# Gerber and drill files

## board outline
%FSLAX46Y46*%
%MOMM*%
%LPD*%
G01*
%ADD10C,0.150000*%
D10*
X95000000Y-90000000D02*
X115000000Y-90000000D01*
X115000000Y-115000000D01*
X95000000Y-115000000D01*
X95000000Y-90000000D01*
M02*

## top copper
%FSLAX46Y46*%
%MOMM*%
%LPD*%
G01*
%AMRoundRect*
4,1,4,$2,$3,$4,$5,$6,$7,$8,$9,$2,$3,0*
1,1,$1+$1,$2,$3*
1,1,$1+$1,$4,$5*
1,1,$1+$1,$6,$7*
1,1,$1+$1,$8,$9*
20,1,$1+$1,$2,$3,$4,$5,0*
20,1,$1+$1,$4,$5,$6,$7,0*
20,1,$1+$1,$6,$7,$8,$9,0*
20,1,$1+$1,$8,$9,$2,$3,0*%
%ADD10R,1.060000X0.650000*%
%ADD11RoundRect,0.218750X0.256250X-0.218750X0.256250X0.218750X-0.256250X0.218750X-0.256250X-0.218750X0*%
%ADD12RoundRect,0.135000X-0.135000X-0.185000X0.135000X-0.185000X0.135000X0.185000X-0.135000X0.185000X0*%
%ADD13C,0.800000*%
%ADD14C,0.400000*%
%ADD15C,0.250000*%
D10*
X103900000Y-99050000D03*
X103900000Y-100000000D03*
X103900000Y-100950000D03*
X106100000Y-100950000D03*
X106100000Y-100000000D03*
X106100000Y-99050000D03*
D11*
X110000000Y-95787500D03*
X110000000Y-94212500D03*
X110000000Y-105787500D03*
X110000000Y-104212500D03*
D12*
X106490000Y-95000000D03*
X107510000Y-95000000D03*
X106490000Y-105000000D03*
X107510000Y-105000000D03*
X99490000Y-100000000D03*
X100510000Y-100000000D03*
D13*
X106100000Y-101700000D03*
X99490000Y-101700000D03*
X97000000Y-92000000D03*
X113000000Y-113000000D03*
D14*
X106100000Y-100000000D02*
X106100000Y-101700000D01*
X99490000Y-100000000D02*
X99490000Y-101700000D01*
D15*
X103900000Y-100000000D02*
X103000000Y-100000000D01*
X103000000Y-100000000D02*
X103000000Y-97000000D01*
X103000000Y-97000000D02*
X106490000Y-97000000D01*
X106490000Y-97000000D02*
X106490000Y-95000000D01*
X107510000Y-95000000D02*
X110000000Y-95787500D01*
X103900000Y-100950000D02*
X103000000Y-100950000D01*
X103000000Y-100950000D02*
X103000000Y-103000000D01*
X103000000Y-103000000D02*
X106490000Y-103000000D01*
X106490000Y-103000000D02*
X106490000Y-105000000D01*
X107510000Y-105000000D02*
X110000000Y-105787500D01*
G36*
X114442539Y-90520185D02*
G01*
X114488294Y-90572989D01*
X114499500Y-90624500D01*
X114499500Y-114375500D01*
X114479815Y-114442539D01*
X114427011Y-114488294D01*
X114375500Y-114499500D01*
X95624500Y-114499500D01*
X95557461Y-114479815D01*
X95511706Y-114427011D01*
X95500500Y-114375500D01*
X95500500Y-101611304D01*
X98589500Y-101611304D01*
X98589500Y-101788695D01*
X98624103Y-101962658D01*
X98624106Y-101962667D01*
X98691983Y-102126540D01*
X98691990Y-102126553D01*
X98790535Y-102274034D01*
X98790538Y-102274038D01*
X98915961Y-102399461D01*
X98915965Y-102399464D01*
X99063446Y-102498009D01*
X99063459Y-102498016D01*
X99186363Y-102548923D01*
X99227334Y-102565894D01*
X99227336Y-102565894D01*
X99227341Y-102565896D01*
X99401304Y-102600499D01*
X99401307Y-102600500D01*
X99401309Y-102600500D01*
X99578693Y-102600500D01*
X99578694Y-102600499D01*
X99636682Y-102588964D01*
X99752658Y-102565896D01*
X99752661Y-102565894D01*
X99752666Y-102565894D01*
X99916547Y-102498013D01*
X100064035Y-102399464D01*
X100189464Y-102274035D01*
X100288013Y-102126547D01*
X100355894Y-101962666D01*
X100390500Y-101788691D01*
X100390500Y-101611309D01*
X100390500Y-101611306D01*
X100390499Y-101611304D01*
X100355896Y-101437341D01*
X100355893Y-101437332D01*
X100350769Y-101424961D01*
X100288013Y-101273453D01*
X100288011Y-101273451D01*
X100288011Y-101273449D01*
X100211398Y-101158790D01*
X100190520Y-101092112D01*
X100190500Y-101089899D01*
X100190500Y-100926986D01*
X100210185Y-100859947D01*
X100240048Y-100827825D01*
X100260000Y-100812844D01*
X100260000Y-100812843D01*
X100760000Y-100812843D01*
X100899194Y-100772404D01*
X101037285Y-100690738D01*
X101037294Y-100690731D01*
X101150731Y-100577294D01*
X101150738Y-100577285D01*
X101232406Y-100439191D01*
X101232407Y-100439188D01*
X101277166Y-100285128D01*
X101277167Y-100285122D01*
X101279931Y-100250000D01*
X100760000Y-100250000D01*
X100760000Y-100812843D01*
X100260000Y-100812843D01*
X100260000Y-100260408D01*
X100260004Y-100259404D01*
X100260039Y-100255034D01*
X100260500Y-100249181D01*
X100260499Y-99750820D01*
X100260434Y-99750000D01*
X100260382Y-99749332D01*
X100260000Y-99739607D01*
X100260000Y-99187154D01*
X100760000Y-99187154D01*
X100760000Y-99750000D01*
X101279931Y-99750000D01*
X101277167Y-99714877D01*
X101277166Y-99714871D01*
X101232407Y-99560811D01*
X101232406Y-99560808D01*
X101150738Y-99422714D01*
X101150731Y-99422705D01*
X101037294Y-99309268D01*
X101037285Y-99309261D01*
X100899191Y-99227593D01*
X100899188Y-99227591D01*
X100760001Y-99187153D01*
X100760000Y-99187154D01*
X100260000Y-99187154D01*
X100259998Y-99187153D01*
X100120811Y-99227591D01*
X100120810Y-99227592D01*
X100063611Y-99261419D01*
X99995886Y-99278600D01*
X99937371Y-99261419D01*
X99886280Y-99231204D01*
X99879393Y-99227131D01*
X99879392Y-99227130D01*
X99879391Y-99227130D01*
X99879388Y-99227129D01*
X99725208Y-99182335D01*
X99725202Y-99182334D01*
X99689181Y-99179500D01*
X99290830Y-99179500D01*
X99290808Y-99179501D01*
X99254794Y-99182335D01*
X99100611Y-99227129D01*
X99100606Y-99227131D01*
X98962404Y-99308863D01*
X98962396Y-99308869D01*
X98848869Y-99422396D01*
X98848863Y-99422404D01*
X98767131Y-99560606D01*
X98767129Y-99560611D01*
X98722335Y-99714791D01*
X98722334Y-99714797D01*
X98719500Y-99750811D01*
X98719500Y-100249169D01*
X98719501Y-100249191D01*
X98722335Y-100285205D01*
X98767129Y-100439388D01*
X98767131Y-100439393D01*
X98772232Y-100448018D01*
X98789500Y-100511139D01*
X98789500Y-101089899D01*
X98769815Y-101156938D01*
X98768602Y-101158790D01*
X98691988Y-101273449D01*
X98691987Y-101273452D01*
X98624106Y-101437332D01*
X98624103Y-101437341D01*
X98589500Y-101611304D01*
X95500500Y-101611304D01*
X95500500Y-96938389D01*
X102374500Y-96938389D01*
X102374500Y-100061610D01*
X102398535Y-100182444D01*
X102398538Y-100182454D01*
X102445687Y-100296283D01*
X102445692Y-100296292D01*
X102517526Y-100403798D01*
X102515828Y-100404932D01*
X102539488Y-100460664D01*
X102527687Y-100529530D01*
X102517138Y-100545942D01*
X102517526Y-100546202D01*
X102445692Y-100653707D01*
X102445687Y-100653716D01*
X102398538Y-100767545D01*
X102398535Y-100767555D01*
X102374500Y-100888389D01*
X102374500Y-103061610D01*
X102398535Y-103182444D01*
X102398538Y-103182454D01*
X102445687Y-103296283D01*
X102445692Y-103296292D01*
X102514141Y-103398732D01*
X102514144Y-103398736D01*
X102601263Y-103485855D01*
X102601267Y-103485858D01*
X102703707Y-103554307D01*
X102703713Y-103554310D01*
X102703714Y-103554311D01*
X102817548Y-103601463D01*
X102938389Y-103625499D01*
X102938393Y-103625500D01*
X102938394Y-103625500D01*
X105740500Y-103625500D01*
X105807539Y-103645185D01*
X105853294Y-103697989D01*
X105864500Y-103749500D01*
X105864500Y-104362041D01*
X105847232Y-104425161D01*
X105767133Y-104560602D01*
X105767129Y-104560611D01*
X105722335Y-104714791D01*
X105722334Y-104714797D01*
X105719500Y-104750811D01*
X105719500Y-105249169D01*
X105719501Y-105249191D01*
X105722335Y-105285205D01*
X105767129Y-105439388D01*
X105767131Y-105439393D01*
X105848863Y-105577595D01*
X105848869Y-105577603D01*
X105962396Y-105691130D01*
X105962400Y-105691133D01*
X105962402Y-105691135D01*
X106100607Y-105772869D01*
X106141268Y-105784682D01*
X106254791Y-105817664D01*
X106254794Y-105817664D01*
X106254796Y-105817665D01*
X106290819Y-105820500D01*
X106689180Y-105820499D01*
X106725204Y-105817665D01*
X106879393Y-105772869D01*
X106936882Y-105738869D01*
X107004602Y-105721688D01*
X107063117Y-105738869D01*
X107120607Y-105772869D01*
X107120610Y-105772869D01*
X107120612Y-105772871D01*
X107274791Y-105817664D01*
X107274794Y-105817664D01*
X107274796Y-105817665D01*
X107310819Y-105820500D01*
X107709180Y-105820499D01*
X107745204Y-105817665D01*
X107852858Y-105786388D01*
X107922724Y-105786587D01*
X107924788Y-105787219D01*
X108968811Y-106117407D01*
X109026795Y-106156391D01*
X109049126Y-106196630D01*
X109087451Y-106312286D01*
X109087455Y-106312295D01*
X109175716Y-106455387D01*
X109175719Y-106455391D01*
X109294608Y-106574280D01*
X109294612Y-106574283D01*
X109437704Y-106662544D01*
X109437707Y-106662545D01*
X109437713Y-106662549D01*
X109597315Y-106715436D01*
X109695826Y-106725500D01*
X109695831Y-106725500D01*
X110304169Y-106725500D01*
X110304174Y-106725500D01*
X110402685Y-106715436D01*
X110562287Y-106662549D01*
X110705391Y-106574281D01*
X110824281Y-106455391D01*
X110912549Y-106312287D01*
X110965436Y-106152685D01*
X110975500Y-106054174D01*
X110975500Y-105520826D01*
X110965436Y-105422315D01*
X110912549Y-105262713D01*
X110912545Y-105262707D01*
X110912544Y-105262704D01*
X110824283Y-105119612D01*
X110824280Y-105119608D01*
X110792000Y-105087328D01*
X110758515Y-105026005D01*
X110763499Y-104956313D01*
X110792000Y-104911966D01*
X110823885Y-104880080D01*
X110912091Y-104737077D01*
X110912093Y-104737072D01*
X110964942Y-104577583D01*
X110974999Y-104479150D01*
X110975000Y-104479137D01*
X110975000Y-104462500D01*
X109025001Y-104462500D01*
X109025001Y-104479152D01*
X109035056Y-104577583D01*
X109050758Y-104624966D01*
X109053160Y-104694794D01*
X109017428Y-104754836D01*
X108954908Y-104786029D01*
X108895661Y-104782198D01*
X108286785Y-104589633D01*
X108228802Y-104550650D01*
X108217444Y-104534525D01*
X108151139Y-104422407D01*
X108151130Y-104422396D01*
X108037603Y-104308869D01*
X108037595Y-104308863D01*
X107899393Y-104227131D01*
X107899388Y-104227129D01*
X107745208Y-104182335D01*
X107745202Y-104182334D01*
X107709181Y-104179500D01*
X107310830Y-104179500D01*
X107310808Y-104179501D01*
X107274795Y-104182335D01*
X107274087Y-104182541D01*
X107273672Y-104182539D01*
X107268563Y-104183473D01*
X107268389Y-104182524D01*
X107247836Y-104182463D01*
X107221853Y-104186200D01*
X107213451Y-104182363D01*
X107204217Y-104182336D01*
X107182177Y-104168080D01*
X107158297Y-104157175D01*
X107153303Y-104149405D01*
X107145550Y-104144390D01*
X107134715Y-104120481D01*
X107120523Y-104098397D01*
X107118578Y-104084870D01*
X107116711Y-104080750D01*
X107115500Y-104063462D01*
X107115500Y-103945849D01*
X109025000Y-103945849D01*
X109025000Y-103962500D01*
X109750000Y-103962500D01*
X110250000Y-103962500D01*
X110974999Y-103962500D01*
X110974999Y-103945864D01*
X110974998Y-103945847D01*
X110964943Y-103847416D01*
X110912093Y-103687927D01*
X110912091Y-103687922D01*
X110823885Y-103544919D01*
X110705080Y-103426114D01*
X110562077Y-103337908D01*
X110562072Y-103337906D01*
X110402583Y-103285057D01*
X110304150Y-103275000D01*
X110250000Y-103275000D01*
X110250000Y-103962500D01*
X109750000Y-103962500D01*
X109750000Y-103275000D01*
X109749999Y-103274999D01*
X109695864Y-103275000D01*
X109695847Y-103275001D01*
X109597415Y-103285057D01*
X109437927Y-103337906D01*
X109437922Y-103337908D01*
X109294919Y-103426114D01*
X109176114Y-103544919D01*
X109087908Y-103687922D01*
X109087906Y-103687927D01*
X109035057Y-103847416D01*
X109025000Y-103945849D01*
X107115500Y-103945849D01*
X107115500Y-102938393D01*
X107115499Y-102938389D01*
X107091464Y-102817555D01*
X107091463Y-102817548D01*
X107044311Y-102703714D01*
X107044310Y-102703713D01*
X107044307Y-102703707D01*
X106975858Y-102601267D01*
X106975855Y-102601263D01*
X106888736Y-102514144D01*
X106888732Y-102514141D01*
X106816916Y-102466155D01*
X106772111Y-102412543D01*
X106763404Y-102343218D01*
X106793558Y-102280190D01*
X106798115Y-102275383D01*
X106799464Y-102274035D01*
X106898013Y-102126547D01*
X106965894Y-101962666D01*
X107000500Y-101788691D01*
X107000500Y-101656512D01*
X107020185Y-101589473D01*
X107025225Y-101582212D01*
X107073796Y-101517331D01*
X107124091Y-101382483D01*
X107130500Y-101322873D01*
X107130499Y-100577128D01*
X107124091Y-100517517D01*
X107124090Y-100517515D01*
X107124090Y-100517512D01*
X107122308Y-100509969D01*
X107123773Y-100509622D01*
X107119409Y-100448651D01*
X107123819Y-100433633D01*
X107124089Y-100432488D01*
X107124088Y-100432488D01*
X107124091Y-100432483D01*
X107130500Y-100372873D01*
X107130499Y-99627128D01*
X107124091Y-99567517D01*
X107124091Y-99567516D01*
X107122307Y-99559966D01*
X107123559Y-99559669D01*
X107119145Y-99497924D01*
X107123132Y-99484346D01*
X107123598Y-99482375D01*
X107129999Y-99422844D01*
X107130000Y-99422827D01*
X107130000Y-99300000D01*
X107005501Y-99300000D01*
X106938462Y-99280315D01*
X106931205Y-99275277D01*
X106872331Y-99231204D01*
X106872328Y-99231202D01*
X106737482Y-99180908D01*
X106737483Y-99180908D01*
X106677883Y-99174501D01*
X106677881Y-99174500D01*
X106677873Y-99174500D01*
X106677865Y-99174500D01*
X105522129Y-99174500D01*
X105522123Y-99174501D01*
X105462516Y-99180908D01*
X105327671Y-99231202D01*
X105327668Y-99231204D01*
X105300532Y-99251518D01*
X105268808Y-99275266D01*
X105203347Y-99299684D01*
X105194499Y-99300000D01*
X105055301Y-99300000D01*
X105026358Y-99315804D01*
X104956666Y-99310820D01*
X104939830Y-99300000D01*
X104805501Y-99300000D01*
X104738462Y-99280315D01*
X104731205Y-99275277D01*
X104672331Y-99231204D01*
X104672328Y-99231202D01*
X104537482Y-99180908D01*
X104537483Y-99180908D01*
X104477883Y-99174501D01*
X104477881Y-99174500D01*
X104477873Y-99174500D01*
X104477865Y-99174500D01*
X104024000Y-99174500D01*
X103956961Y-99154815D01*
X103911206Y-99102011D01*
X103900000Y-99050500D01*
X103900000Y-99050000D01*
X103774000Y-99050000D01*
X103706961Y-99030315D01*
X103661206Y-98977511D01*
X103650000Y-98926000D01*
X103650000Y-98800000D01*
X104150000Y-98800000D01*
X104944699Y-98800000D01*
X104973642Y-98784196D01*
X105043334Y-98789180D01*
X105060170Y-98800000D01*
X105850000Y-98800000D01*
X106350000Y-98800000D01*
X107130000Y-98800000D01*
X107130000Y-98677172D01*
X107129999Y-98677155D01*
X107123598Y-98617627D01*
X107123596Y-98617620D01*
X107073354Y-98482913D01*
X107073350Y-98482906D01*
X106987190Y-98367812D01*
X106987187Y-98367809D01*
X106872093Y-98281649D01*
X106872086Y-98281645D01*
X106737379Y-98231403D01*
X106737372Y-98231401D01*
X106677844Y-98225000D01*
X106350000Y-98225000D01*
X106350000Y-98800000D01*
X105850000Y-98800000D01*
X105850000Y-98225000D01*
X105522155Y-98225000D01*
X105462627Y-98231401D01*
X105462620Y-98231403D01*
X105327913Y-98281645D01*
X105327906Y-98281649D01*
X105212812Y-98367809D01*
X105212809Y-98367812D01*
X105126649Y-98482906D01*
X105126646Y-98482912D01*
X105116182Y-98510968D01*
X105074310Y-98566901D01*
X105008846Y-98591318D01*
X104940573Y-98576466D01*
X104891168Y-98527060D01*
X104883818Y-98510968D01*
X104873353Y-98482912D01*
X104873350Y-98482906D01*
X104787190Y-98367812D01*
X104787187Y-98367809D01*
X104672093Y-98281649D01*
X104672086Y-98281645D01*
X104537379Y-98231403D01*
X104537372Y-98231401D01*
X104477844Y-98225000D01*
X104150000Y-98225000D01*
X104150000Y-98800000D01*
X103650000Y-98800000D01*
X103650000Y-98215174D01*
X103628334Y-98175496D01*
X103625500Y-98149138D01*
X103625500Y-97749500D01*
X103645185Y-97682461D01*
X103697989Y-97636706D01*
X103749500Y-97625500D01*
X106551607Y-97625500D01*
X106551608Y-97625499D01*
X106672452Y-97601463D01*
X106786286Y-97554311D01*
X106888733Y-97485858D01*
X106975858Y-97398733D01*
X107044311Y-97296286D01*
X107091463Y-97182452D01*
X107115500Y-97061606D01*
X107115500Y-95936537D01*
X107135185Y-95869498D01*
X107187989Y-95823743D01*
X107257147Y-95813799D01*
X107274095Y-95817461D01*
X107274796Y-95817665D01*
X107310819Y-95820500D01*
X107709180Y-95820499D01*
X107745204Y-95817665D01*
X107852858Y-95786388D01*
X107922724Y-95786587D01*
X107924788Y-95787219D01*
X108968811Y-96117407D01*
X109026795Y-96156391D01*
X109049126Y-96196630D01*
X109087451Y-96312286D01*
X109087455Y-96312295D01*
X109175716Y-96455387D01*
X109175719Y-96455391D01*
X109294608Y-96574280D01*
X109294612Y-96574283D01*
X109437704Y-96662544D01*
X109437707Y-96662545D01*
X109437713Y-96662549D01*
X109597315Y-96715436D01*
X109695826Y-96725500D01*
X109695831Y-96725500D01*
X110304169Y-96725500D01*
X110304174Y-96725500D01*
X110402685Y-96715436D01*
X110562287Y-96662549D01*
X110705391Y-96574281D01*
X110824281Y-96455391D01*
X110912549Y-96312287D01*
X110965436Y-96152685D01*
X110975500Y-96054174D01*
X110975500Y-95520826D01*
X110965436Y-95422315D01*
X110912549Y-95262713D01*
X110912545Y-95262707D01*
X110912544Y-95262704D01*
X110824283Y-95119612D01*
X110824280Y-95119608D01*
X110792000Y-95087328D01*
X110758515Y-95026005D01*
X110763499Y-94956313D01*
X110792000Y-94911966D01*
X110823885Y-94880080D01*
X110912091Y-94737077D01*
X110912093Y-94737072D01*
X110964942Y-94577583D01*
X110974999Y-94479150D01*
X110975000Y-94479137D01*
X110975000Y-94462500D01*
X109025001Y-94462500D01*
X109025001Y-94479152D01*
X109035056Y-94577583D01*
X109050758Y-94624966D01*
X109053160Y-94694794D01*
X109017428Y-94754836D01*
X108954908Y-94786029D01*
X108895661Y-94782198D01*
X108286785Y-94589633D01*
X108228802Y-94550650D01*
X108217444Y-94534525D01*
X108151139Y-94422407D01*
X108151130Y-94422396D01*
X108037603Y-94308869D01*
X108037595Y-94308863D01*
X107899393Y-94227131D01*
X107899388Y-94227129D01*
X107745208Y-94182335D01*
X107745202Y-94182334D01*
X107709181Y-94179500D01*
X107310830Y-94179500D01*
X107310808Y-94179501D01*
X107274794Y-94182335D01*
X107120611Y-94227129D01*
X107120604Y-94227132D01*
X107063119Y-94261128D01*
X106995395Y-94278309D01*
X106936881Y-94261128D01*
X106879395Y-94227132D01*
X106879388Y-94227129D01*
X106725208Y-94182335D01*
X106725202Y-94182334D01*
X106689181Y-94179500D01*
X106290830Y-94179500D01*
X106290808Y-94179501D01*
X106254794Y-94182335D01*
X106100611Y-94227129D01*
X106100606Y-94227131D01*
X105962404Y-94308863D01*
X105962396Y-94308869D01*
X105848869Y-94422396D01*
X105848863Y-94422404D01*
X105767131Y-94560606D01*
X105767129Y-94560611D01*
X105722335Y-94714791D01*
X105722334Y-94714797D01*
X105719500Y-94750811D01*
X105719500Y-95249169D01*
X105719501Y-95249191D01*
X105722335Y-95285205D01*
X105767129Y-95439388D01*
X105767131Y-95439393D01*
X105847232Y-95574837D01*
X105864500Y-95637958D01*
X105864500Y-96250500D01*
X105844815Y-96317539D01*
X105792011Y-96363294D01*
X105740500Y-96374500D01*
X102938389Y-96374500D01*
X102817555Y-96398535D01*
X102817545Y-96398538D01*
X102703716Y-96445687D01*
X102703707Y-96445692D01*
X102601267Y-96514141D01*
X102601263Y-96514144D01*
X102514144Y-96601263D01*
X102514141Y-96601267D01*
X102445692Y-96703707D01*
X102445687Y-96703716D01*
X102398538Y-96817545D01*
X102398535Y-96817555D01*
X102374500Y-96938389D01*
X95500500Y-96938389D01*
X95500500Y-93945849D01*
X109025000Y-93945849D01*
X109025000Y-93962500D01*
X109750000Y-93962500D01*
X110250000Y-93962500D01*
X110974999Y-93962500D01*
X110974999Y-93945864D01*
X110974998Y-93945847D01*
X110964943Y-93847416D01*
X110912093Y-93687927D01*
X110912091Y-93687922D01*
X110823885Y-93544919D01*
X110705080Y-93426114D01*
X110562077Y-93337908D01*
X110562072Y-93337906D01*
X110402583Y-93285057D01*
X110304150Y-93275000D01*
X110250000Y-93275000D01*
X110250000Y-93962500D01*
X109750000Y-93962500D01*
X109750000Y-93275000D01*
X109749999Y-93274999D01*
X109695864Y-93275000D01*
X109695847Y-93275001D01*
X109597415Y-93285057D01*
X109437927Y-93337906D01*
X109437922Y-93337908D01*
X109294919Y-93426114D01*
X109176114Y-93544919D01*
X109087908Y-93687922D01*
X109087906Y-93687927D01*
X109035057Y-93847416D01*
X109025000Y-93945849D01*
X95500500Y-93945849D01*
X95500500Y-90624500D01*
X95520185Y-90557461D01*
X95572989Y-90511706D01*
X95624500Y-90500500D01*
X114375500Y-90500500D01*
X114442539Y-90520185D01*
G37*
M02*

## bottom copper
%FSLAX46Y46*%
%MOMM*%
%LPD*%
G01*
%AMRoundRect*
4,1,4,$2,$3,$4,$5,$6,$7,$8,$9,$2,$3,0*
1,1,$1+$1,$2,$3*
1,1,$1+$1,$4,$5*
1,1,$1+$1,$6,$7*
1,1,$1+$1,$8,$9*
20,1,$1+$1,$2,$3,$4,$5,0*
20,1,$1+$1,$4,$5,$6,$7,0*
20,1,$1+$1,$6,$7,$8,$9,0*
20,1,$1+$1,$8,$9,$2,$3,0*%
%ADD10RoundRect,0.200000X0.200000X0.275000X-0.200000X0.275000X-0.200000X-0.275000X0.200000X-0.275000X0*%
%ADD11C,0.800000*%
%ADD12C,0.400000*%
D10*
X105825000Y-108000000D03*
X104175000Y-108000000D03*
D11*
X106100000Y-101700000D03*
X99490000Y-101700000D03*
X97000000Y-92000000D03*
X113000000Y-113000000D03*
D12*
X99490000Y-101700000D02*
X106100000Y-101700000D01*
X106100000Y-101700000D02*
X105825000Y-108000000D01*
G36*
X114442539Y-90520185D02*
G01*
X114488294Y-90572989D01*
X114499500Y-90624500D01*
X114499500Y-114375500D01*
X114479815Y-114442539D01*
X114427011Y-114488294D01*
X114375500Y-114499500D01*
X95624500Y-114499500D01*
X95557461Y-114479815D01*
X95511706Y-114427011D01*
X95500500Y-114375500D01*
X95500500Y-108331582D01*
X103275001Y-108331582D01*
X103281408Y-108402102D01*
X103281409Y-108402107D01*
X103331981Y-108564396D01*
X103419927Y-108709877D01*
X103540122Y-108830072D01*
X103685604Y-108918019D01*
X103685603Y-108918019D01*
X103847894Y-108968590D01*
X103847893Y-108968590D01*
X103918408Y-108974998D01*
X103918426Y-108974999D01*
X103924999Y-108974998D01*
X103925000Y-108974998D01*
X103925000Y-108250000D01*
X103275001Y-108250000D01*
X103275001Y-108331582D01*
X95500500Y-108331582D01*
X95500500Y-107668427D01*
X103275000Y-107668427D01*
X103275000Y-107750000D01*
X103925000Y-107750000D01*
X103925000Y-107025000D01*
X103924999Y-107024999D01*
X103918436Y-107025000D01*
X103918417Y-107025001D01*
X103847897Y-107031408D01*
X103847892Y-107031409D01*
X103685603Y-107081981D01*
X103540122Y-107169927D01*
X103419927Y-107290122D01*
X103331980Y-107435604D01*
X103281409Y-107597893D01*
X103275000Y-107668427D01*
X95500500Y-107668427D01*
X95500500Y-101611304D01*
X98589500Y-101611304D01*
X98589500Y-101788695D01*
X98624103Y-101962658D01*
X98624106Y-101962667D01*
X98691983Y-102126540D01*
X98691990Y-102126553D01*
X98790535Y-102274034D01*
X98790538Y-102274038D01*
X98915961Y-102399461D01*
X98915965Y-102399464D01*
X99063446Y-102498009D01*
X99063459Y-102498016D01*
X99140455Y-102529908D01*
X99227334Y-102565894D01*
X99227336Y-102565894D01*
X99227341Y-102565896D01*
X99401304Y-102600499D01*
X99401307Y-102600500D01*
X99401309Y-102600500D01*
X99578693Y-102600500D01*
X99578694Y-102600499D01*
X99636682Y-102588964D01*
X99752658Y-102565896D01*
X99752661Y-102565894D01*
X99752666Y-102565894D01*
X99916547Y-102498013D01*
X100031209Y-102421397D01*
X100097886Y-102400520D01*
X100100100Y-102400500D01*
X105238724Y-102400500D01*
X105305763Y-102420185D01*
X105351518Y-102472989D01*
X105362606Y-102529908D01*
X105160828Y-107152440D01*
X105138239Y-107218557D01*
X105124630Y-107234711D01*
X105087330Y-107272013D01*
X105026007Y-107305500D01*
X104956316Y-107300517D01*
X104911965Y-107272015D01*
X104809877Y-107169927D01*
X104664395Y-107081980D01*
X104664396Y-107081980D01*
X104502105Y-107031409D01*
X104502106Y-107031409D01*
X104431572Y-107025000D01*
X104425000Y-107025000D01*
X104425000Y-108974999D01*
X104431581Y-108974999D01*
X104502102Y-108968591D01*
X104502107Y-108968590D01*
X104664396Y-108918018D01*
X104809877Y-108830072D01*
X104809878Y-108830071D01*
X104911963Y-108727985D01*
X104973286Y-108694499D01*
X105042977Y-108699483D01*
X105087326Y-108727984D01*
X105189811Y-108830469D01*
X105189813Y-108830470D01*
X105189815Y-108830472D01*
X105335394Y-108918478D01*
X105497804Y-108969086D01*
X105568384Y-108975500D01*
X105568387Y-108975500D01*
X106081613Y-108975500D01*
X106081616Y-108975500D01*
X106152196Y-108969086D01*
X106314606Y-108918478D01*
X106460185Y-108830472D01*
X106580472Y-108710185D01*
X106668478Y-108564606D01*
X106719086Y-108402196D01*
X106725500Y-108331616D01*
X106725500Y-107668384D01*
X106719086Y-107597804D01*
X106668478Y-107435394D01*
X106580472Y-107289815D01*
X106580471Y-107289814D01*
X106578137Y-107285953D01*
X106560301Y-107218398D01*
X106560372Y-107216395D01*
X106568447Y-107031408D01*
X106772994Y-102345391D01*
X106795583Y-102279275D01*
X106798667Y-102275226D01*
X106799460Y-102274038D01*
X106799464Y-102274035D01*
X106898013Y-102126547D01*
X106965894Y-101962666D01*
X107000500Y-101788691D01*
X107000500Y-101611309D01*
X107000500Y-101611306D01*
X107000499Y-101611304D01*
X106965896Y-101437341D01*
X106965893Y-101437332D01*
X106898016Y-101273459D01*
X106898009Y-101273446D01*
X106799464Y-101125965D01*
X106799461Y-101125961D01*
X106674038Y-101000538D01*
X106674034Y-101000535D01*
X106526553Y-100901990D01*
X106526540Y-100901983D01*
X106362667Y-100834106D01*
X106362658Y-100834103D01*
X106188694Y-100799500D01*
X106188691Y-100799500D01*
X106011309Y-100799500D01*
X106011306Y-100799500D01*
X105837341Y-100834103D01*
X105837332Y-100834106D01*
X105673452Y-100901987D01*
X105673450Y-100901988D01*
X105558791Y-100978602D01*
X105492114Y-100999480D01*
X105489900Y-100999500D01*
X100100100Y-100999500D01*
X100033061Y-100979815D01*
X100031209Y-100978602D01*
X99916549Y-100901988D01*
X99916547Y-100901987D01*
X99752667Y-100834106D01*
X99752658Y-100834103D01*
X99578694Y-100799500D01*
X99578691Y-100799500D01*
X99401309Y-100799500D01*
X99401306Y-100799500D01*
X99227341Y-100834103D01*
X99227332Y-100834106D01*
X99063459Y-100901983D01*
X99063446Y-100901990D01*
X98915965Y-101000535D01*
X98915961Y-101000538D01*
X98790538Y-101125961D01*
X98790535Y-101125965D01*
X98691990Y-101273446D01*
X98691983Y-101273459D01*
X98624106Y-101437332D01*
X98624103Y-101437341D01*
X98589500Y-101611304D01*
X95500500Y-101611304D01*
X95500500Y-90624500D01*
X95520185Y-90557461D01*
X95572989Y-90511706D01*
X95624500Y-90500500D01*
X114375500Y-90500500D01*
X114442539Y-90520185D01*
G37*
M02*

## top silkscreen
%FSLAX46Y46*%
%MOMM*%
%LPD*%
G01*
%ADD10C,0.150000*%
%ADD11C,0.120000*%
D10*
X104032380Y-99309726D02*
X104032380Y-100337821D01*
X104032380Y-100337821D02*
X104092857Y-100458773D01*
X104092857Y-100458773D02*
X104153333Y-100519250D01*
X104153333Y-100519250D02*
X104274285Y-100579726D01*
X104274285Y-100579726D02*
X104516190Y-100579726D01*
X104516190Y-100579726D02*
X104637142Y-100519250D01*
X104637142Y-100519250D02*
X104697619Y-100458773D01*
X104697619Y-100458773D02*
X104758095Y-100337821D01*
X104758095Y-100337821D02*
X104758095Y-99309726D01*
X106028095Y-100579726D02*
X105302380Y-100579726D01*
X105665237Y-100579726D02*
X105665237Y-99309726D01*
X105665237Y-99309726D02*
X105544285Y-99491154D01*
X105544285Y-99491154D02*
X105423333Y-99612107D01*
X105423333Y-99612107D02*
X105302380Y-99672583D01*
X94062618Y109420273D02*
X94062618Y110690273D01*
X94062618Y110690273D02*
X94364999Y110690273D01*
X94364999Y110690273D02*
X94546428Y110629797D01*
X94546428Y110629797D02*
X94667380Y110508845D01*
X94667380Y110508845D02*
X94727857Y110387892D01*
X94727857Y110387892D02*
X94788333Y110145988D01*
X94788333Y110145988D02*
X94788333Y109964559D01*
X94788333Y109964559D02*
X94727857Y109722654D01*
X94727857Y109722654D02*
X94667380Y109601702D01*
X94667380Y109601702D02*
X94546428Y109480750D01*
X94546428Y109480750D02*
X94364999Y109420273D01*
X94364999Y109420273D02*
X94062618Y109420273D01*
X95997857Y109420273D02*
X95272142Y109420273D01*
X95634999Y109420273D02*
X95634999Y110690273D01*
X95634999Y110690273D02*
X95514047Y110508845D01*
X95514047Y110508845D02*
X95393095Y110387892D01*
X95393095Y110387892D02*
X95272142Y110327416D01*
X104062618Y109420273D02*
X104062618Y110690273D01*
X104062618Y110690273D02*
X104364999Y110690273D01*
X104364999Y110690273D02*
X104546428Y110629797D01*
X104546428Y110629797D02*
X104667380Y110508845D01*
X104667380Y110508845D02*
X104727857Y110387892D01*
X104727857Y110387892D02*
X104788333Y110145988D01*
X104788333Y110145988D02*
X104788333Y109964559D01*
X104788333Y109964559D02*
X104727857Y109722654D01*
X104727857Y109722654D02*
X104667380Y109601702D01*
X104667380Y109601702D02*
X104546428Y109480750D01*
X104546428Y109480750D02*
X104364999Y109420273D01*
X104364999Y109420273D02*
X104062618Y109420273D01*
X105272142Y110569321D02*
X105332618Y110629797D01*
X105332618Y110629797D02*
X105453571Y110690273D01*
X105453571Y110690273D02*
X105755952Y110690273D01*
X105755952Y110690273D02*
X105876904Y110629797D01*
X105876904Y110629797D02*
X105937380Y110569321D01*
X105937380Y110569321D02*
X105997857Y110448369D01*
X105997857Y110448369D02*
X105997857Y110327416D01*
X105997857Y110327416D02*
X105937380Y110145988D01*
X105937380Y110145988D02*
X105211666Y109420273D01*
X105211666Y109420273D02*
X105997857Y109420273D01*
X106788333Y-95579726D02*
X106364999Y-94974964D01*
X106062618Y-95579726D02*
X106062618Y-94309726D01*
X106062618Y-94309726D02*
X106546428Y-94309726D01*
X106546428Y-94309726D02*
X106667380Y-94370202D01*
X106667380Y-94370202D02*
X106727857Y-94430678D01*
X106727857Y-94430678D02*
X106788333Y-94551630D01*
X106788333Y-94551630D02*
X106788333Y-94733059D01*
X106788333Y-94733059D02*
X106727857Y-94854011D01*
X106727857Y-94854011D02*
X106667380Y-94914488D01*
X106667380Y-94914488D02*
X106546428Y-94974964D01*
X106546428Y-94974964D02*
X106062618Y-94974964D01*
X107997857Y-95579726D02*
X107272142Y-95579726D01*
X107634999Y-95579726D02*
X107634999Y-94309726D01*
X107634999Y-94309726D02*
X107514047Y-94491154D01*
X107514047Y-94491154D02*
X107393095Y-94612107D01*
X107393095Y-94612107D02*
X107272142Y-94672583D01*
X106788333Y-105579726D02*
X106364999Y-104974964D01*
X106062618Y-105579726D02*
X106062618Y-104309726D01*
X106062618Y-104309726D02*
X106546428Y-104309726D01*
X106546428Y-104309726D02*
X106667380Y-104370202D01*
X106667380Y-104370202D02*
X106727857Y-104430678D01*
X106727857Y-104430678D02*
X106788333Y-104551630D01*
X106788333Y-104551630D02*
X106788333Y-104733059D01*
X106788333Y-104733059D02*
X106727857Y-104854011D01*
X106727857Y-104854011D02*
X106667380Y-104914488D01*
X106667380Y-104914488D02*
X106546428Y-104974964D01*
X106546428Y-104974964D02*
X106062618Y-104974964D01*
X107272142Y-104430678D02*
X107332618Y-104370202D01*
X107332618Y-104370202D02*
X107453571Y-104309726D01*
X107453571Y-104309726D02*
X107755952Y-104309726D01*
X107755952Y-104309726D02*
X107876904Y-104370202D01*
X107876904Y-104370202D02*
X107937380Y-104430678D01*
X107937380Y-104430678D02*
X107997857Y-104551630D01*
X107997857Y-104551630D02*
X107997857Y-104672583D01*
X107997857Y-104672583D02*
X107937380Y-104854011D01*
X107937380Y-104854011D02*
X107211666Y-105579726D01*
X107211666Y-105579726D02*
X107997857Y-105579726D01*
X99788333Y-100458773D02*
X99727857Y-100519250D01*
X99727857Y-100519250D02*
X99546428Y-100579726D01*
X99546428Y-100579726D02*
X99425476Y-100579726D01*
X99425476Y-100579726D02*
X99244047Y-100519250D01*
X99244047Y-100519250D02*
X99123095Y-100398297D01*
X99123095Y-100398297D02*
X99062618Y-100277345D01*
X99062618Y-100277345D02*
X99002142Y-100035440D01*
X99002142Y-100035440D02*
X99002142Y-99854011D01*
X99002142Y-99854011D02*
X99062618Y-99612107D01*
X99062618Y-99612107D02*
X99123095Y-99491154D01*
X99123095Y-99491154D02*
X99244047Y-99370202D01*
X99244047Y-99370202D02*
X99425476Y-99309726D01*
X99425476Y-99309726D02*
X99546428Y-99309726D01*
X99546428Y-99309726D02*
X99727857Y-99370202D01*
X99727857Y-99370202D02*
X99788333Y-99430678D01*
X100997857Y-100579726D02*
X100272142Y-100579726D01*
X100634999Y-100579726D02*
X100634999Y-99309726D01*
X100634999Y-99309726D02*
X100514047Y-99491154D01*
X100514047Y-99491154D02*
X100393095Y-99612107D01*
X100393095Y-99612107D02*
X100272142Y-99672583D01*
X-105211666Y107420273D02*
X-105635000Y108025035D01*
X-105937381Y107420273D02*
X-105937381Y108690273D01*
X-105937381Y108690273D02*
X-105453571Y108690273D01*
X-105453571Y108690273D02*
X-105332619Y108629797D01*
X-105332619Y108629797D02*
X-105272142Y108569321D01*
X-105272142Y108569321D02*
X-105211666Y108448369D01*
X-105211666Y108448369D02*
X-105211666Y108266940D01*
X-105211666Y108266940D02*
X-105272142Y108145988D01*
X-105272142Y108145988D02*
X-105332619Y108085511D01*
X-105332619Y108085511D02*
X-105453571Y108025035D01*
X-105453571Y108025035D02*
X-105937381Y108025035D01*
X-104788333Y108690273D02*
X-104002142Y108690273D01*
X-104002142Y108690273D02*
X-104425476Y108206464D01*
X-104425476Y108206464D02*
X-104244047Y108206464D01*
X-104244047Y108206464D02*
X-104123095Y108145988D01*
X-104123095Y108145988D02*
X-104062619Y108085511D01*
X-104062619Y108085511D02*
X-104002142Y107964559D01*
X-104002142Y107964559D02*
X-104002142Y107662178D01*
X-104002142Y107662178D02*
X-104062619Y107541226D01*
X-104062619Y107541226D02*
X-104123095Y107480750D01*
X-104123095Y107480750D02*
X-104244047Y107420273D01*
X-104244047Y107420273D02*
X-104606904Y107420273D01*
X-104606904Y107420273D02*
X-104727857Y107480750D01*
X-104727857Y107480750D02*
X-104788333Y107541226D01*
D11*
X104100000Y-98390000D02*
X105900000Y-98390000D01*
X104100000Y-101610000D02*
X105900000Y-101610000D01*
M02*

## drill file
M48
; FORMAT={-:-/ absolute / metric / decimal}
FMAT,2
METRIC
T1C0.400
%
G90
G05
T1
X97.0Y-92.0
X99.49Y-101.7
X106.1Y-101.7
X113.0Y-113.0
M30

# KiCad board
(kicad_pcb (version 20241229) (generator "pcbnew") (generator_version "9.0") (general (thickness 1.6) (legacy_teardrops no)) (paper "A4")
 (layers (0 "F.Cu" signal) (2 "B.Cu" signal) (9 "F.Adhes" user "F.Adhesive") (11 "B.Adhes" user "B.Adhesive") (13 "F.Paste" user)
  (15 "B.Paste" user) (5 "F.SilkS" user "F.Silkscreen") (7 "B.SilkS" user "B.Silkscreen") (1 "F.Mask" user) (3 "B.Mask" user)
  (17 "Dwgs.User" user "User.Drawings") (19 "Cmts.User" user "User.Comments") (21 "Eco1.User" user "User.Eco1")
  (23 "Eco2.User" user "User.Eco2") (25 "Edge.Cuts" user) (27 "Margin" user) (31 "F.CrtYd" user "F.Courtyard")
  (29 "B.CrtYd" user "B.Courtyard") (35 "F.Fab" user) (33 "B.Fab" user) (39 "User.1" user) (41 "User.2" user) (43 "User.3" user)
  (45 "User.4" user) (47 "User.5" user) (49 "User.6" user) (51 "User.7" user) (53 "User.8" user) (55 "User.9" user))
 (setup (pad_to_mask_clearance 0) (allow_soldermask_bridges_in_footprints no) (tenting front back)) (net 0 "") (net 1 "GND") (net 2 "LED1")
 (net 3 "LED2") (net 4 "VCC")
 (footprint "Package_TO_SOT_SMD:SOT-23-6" (layer "F.Cu") (at 105 100)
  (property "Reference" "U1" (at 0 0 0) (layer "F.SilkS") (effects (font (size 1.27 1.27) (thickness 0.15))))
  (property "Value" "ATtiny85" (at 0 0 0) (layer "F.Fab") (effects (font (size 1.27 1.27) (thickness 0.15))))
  (fp_line (start -0.9 -1.61) (end 0.9 -1.61) (stroke (width 0.12) (type solid)) (layer "F.SilkS"))
  (fp_line (start -0.9 1.61) (end 0.9 1.61) (stroke (width 0.12) (type solid)) (layer "F.SilkS"))
  (pad "1" smd rect (at -1.1 -0.95) (size 1.06 0.65) (layers "F.Cu" "F.Mask" "F.Paste") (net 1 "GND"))
  (pad "2" smd rect (at -1.1 0) (size 1.06 0.65) (layers "F.Cu" "F.Mask" "F.Paste") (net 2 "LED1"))
  (pad "3" smd rect (at -1.1 0.95) (size 1.06 0.65) (layers "F.Cu" "F.Mask" "F.Paste") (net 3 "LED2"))
  (pad "4" smd rect (at 1.1 0.95) (size 1.06 0.65) (layers "F.Cu" "F.Mask" "F.Paste") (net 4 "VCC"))
  (pad "5" smd rect (at 1.1 0) (size 1.06 0.65) (layers "F.Cu" "F.Mask" "F.Paste") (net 4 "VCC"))
  (pad "6" smd rect (at 1.1 -0.95) (size 1.06 0.65) (layers "F.Cu" "F.Mask" "F.Paste") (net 1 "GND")))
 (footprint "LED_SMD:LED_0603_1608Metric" (layer "F.Cu") (at 110 95 90)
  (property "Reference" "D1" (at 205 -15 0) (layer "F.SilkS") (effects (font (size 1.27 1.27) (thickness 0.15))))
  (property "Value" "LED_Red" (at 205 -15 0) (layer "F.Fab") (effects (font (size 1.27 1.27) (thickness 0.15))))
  (pad "1" smd roundrect (at -0.7875 0 90) (size 0.875 0.95) (layers "F.Cu" "F.Mask" "F.Paste") (roundrect_rratio 0.25) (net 2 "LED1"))
  (pad "2" smd roundrect (at 0.7875 0 90) (size 0.875 0.95) (layers "F.Cu" "F.Mask" "F.Paste") (roundrect_rratio 0.25) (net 1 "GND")))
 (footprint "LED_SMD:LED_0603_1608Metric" (layer "F.Cu") (at 110 105 90)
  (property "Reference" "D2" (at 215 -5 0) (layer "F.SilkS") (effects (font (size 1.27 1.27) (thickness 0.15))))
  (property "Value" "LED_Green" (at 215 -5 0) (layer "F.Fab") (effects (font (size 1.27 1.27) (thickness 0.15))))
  (pad "1" smd roundrect (at -0.7875 0 90) (size 0.875 0.95) (layers "F.Cu" "F.Mask" "F.Paste") (roundrect_rratio 0.25) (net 3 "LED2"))
  (pad "2" smd roundrect (at 0.7875 0 90) (size 0.875 0.95) (layers "F.Cu" "F.Mask" "F.Paste") (roundrect_rratio 0.25) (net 1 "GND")))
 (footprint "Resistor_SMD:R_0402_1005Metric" (layer "F.Cu") (at 107 95)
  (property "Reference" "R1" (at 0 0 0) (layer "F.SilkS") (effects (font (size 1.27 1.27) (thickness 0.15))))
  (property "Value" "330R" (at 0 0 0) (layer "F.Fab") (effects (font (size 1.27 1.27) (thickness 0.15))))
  (pad "1" smd roundrect (at -0.51 0) (size 0.54 0.64) (layers "F.Cu" "F.Mask" "F.Paste") (roundrect_rratio 0.25) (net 2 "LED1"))
  (pad "2" smd roundrect (at 0.51 0) (size 0.54 0.64) (layers "F.Cu" "F.Mask" "F.Paste") (roundrect_rratio 0.25) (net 2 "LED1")))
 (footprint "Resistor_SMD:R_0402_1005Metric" (layer "F.Cu") (at 107 105)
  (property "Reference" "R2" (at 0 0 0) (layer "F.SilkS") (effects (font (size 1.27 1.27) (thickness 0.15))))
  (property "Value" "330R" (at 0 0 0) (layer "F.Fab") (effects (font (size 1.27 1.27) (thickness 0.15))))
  (pad "1" smd roundrect (at -0.51 0) (size 0.54 0.64) (layers "F.Cu" "F.Mask" "F.Paste") (roundrect_rratio 0.25) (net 3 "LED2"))
  (pad "2" smd roundrect (at 0.51 0) (size 0.54 0.64) (layers "F.Cu" "F.Mask" "F.Paste") (roundrect_rratio 0.25) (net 3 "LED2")))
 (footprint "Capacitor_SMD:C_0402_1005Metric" (layer "F.Cu") (at 100 100)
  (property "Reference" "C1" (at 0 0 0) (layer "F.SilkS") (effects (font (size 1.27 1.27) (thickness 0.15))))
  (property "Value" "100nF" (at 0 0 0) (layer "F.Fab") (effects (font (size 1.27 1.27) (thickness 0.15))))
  (pad "1" smd roundrect (at -0.51 0) (size 0.54 0.64) (layers "F.Cu" "F.Mask" "F.Paste") (roundrect_rratio 0.25) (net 4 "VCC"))
  (pad "2" smd roundrect (at 0.51 0) (size 0.54 0.64) (layers "F.Cu" "F.Mask" "F.Paste") (roundrect_rratio 0.25) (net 1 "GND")))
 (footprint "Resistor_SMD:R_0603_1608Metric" (layer "B.Cu") (at 105 108 180)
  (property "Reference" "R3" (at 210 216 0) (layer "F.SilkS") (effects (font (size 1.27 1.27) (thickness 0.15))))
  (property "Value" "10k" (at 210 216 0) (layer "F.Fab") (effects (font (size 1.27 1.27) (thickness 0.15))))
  (pad "1" smd roundrect (at -0.825 0 180) (size 0.8 0.95) (layers "B.Cu" "B.Mask" "B.Paste") (roundrect_rratio 0.25) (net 4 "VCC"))
  (pad "2" smd roundrect (at 0.825 0 180) (size 0.8 0.95) (layers "B.Cu" "B.Mask" "B.Paste") (roundrect_rratio 0.25) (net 1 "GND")))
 (gr_rect (start 95 90) (end 115 115) (stroke (width 0.15) (type solid)) (fill no) (layer "Edge.Cuts"))
 (segment (start 106.1 100) (end 106.1 101.7) (width 0.4) (layer "F.Cu") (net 4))
 (segment (start 99.49 100) (end 99.49 101.7) (width 0.4) (layer "F.Cu") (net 4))
 (via (at 106.1 101.7) (size 0.8) (drill 0.4) (layers "F.Cu" "B.Cu") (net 4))
 (via (at 99.49 101.7) (size 0.8) (drill 0.4) (layers "F.Cu" "B.Cu") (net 4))
 (segment (start 99.49 101.7) (end 106.1 101.7) (width 0.4) (layer "B.Cu") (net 4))
 (segment (start 106.1 101.7) (end 105.825 108) (width 0.4) (layer "B.Cu") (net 4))
 (via (at 97 92) (size 0.8) (drill 0.4) (layers "F.Cu" "B.Cu") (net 1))
 (via (at 113 113) (size 0.8) (drill 0.4) (layers "F.Cu" "B.Cu") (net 1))
 (segment (start 103.9 100) (end 103 100) (width 0.25) (layer "F.Cu") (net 2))
 (segment (start 103 100) (end 103 97) (width 0.25) (layer "F.Cu") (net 2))
 (segment (start 103 97) (end 106.49 97) (width 0.25) (layer "F.Cu") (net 2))
 (segment (start 106.49 97) (end 106.49 95) (width 0.25) (layer "F.Cu") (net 2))
 (segment (start 107.51 95) (end 110 95.7875) (width 0.25) (layer "F.Cu") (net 2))
 (segment (start 103.9 100.95) (end 103 100.95) (width 0.25) (layer "F.Cu") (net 3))
 (segment (start 103 100.95) (end 103 103) (width 0.25) (layer "F.Cu") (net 3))
 (segment (start 103 103) (end 106.49 103) (width 0.25) (layer "F.Cu") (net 3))
 (segment (start 106.49 103) (end 106.49 105) (width 0.25) (layer "F.Cu") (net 3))
 (segment (start 107.51 105) (end 110 105.7875) (width 0.25) (layer "F.Cu") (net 3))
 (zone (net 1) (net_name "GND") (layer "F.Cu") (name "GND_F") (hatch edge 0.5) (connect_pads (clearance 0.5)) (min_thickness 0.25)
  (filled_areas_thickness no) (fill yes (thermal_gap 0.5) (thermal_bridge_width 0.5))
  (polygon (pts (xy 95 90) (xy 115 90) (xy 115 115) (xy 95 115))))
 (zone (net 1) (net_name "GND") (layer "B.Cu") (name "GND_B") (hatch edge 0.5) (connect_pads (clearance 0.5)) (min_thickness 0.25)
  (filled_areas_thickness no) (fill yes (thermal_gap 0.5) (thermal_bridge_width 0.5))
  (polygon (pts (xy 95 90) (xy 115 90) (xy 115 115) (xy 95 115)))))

